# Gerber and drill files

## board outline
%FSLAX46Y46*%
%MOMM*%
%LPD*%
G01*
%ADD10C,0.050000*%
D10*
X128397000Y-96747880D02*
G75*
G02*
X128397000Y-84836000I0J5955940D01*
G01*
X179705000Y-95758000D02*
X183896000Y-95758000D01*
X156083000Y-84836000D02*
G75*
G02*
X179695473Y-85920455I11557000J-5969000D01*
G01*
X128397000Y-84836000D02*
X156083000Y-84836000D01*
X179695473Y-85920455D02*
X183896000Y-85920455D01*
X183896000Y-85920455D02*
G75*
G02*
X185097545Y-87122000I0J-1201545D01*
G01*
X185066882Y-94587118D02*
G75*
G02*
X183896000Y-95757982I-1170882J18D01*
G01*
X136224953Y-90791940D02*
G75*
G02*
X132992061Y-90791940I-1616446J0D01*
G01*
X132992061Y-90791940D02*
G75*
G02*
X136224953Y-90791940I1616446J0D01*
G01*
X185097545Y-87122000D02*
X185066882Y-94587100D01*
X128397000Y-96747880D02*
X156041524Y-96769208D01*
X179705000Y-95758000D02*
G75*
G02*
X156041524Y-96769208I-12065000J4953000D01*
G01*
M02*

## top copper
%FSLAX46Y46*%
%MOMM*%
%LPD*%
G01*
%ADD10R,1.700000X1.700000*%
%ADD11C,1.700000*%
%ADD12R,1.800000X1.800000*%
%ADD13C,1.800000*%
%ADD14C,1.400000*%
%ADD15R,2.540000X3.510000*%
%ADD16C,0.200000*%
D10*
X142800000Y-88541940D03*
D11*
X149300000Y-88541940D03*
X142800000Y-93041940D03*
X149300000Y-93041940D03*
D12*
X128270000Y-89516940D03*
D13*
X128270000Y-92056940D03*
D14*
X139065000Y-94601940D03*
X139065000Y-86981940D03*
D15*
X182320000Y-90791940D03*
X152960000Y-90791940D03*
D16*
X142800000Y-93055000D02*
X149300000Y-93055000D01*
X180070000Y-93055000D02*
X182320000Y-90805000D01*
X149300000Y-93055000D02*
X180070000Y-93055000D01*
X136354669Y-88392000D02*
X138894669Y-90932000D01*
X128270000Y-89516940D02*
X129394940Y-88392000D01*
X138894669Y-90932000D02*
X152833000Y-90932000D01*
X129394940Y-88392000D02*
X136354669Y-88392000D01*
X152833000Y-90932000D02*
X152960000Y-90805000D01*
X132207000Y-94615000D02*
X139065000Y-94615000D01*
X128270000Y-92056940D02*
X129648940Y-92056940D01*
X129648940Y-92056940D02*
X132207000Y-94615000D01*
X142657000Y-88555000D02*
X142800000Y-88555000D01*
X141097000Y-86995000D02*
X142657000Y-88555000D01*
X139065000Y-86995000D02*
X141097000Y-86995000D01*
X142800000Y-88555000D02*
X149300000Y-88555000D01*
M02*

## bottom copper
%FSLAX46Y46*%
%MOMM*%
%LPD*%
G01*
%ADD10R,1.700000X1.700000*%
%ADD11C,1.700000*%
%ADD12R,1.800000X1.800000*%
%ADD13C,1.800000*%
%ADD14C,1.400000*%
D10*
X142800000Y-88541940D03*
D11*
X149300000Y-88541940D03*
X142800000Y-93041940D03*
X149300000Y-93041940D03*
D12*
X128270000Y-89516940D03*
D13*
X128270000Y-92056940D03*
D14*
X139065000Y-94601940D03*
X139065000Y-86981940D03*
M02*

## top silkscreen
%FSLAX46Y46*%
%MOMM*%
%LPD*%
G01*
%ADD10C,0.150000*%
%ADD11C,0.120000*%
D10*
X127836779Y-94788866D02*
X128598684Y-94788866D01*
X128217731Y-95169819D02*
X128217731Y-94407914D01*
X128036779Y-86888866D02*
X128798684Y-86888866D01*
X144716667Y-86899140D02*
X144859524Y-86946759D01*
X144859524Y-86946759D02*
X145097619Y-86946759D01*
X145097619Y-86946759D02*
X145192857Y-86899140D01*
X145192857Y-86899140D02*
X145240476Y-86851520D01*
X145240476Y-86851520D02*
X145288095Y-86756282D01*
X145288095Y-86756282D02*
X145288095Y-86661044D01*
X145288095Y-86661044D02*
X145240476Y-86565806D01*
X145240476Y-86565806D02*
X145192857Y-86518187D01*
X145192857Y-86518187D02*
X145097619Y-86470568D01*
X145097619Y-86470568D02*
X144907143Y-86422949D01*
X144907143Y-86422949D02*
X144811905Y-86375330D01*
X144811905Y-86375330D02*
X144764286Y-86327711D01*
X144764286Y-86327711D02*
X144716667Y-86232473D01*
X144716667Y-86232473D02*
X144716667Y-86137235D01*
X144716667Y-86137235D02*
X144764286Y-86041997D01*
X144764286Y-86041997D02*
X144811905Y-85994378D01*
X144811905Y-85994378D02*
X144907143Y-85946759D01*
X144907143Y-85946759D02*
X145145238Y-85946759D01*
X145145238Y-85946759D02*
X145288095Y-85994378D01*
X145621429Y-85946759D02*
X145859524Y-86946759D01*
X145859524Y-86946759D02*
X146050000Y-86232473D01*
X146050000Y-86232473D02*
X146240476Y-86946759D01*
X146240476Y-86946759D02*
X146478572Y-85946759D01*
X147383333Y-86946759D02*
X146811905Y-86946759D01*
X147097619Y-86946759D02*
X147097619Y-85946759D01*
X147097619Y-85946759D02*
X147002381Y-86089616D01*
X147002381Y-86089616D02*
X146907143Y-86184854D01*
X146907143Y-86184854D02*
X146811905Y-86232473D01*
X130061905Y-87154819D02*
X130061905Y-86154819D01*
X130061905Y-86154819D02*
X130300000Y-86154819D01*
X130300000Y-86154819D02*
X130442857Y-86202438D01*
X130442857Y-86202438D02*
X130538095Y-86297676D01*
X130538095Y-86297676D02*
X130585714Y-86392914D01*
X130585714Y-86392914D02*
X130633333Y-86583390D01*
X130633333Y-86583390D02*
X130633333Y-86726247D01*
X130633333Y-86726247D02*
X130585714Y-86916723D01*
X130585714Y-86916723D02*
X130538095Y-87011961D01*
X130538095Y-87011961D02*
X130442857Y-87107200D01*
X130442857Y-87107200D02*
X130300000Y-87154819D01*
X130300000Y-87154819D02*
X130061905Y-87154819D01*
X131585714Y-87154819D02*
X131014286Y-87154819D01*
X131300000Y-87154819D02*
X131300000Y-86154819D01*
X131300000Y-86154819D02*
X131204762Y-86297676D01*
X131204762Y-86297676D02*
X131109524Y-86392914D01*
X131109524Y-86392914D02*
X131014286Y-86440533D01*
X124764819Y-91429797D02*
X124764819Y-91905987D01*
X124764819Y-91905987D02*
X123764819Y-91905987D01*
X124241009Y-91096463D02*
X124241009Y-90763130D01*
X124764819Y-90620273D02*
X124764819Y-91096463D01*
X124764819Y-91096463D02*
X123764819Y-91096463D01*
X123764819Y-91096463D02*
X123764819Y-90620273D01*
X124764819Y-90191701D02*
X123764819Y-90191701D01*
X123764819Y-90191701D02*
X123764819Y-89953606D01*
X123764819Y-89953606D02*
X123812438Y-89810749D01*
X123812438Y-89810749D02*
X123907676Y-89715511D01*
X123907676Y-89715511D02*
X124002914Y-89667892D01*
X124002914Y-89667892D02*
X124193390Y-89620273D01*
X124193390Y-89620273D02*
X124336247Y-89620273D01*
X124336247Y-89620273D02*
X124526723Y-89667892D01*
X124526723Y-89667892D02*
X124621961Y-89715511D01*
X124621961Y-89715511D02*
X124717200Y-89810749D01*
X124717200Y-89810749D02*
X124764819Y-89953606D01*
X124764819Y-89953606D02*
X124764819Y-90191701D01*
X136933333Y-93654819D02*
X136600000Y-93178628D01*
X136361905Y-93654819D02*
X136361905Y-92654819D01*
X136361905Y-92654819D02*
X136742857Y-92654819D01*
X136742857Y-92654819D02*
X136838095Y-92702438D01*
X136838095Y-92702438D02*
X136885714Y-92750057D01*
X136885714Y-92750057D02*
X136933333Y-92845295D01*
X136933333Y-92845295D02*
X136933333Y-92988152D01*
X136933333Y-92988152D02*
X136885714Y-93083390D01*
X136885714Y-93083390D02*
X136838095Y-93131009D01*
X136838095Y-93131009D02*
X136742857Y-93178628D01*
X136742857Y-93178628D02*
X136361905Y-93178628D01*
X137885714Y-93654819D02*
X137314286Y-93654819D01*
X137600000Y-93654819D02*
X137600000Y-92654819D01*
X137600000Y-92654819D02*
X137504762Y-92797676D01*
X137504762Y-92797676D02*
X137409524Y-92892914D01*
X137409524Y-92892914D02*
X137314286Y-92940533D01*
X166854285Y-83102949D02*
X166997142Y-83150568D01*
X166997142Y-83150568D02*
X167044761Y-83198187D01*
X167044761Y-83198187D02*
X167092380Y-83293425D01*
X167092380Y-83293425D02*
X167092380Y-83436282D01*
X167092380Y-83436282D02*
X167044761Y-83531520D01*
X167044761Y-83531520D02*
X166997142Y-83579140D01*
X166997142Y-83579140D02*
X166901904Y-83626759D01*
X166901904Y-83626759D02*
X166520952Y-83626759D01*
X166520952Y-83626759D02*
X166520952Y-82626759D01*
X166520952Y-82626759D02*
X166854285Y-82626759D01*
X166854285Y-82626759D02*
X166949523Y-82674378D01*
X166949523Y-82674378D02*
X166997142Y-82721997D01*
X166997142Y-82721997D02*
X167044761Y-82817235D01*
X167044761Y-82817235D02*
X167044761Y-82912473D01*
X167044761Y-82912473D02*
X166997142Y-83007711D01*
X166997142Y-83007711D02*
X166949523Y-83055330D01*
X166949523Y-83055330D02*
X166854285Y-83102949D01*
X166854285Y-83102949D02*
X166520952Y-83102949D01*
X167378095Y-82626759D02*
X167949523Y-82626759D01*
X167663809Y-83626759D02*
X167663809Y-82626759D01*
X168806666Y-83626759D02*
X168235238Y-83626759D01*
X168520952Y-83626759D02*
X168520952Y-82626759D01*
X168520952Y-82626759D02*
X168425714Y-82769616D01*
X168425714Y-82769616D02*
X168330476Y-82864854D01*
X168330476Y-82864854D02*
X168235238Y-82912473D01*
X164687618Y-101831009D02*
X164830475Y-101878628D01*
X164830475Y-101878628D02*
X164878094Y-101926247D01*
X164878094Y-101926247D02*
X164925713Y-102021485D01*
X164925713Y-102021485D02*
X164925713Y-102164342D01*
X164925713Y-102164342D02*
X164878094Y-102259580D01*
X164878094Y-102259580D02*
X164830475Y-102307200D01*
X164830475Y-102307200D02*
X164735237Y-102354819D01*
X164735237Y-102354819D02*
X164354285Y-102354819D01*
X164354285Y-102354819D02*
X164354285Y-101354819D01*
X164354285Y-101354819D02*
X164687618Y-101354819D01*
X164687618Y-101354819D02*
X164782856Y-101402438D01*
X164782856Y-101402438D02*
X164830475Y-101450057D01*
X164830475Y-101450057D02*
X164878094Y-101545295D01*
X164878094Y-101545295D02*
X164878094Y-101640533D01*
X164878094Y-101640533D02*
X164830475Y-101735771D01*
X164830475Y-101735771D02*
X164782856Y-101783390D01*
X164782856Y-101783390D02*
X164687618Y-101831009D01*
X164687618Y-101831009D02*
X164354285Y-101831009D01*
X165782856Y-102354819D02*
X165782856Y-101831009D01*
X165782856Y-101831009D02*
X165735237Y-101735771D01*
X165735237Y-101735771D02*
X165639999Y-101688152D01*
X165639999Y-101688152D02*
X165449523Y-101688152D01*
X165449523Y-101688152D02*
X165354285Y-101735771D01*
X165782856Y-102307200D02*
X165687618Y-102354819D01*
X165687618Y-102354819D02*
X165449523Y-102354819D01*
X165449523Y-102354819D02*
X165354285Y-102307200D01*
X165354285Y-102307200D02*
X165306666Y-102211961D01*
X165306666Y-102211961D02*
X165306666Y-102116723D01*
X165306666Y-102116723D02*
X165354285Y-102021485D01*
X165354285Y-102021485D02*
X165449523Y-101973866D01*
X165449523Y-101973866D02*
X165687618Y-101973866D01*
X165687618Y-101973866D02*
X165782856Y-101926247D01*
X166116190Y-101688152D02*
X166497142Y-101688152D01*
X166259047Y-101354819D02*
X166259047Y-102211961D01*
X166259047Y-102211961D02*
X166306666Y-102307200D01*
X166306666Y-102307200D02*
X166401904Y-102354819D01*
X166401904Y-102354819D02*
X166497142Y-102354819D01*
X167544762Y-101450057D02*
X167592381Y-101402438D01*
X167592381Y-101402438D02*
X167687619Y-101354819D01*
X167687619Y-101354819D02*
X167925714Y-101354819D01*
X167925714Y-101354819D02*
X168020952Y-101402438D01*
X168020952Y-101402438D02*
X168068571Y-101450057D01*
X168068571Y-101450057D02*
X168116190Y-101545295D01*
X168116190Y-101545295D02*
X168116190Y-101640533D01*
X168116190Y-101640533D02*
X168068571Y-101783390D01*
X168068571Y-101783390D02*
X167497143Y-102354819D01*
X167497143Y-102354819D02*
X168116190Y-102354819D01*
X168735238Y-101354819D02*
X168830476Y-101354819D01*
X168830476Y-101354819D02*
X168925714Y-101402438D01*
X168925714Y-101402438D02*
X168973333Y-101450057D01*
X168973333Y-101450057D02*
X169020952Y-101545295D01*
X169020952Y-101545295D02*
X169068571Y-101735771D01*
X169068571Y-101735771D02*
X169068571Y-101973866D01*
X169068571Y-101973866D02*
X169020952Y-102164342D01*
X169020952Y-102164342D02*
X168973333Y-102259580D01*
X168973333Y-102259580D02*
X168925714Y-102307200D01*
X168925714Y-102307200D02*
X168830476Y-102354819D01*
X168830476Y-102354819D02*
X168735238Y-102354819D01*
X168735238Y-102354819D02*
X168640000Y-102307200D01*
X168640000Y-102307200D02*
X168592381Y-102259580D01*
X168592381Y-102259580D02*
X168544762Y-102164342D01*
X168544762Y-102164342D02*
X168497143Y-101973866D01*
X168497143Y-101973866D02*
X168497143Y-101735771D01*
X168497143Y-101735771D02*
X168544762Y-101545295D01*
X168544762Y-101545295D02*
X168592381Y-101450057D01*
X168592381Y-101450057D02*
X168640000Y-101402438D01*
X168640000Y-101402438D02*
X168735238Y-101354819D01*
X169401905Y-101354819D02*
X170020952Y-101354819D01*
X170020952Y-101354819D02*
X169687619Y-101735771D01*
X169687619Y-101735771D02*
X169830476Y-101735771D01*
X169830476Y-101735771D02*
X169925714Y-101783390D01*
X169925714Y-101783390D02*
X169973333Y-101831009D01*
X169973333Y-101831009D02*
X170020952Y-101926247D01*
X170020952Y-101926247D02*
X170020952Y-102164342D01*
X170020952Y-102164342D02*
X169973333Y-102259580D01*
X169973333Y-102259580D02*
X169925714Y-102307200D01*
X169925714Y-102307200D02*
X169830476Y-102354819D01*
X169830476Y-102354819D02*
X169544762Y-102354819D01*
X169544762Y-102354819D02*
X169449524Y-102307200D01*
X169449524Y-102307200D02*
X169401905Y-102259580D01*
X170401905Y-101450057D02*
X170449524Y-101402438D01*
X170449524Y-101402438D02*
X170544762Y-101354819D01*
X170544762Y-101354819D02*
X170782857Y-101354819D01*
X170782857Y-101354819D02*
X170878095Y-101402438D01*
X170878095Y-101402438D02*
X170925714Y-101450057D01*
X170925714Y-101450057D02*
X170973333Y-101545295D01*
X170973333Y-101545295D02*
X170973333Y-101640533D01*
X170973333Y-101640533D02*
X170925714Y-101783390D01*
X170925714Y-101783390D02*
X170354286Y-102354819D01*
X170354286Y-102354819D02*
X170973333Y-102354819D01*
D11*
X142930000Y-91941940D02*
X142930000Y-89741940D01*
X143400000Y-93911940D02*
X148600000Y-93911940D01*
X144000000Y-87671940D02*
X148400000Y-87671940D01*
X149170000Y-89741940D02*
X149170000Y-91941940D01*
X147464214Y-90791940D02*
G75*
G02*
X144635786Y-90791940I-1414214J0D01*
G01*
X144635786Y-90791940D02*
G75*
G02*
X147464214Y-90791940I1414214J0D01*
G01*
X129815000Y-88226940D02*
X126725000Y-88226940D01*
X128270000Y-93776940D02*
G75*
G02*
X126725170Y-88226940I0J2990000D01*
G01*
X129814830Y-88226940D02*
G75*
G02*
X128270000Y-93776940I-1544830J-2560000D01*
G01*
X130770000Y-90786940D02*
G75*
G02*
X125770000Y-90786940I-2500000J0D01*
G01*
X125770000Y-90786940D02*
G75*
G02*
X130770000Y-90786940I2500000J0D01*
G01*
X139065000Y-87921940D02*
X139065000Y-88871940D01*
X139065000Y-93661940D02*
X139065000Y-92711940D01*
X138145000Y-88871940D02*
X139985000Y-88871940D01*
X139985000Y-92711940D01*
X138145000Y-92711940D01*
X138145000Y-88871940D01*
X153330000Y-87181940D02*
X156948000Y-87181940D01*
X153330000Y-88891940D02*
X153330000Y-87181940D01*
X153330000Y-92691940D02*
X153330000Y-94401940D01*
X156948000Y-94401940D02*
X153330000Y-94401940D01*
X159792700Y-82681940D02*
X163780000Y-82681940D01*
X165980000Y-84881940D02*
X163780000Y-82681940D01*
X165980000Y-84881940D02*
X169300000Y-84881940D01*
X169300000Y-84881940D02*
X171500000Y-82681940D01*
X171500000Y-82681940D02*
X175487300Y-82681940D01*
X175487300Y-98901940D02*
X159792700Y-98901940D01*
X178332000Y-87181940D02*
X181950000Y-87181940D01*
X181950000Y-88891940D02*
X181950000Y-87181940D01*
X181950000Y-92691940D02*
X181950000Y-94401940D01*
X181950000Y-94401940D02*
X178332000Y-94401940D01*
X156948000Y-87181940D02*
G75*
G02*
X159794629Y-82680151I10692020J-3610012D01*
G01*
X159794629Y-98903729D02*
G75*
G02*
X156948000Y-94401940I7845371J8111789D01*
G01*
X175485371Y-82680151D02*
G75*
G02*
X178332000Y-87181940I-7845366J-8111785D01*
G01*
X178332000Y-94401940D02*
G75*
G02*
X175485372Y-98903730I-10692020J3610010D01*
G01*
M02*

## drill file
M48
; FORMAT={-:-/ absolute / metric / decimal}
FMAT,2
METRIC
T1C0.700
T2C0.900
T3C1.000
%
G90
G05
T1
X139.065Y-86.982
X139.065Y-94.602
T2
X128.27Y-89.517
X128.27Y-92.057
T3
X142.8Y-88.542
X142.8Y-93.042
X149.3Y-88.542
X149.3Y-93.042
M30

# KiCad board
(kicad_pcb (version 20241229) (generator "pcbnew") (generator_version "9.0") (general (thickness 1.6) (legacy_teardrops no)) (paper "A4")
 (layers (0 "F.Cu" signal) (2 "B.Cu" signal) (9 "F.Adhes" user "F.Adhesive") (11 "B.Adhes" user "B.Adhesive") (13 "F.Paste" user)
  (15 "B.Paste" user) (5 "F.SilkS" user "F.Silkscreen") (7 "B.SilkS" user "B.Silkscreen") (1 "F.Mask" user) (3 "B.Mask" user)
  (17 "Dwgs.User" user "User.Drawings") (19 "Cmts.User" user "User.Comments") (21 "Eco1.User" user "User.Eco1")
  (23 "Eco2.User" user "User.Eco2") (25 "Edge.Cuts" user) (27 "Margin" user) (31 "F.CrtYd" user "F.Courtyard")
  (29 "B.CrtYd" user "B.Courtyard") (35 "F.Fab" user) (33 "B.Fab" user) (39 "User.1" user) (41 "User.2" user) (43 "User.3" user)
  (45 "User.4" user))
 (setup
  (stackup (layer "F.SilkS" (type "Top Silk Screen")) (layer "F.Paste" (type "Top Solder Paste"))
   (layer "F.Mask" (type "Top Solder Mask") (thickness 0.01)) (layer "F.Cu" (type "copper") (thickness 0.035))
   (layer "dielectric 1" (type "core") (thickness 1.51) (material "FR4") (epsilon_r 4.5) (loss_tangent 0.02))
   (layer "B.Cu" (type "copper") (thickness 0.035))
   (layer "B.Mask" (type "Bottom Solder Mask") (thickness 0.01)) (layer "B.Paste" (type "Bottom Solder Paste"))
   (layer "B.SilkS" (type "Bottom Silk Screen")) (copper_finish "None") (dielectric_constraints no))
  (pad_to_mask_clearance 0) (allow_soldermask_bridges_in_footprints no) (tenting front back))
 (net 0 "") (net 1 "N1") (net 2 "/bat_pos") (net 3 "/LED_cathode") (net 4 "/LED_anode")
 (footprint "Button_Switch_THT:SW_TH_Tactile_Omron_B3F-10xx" (layer "F.Cu") (at 142.8 88.54194)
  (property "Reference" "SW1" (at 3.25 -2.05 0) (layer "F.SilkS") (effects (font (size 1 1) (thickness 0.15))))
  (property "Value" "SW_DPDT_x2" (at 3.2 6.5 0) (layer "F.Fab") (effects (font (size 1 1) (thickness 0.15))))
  (fp_line (start 0.13 3.4) (end 0.13 1.2) (stroke (width 0.12) (type solid)) (layer "F.SilkS"))
  (fp_line (start 0.6 5.37) (end 5.8 5.37) (stroke (width 0.12) (type solid)) (layer "F.SilkS"))
  (fp_line (start 1.2 -0.87) (end 5.6 -0.87) (stroke (width 0.12) (type solid)) (layer "F.SilkS"))
  (fp_line (start 6.37 1.2) (end 6.37 3.4) (stroke (width 0.12) (type solid)) (layer "F.SilkS"))
  (fp_circle (center 3.25 2.25) (end 4.25 3.25) (stroke (width 0.12) (type solid)) (fill no) (layer "F.SilkS"))
  (pad "1" thru_hole rect (at 0 0) (size 1.7 1.7) (drill 1) (layers "*.Cu" "*.Mask") (remove_unused_layers no) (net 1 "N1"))
  (pad "1" thru_hole circle (at 6.5 0) (size 1.7 1.7) (drill 1) (layers "*.Cu" "*.Mask") (remove_unused_layers no) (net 1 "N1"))
  (pad "2" thru_hole circle (at 0 4.5) (size 1.7 1.7) (drill 1) (layers "*.Cu" "*.Mask") (remove_unused_layers no) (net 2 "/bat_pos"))
  (pad "2" thru_hole circle (at 6.5 4.5) (size 1.7 1.7) (drill 1) (layers "*.Cu" "*.Mask") (remove_unused_layers no) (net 2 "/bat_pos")))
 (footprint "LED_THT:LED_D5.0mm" (layer "F.Cu") (at 128.27 89.51694 -90)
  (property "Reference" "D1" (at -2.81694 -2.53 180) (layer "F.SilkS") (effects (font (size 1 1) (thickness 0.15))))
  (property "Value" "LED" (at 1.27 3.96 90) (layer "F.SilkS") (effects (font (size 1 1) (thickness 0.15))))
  (fp_line (start -1.29 -1.545) (end -1.29 1.545) (stroke (width 0.12) (type solid)) (layer "F.SilkS"))
  (fp_arc (start 4.26 0) (mid 2.071779 2.880495) (end -1.29 1.54483) (stroke (width 0.12) (type solid)) (layer "F.SilkS"))
  (fp_arc (start -1.29 -1.54483) (mid 2.071779 -2.880495) (end 4.26 0) (stroke (width 0.12) (type solid)) (layer "F.SilkS"))
  (fp_circle (center 1.27 0) (end 3.77 0) (stroke (width 0.12) (type solid)) (fill no) (layer "F.SilkS"))
  (pad "1" thru_hole rect (at 0 0 270) (size 1.8 1.8) (drill 0.9) (layers "*.Cu" "*.Mask") (remove_unused_layers no) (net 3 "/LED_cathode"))
  (pad "2" thru_hole circle (at 2.54 0 270) (size 1.8 1.8) (drill 0.9) (layers "*.Cu" "*.Mask") (remove_unused_layers no)
   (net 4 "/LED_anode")))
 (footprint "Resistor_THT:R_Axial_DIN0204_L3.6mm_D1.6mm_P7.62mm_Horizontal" (layer "F.Cu") (at 139.065 94.60194 90)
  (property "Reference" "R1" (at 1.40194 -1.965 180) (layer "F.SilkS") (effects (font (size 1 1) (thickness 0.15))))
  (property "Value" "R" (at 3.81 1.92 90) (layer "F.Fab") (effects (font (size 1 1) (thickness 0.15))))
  (fp_line (start 6.68 0) (end 5.73 0) (stroke (width 0.12) (type solid)) (layer "F.SilkS"))
  (fp_line (start 0.94 0) (end 1.89 0) (stroke (width 0.12) (type solid)) (layer "F.SilkS"))
  (fp_rect (start 1.89 -0.92) (end 5.73 0.92) (stroke (width 0.12) (type solid)) (fill no) (layer "F.SilkS"))
  (pad "1" thru_hole circle (at 0 0 90) (size 1.4 1.4) (drill 0.7) (layers "*.Cu" "*.Mask") (remove_unused_layers no) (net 4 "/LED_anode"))
  (pad "2" thru_hole circle (at 7.62 0 90) (size 1.4 1.4) (drill 0.7) (layers "*.Cu" "*.Mask") (remove_unused_layers no) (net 1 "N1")))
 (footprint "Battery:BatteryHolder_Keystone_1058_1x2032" (layer "F.Cu") (at 167.64 90.79194 180)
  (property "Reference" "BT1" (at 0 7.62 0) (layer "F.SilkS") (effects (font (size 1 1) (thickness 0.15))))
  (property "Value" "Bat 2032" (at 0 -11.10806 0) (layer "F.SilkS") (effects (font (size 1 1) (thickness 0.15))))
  (fp_line (start 14.31 3.61) (end 10.692 3.61) (stroke (width 0.12) (type solid)) (layer "F.SilkS"))
  (fp_line (start 14.31 1.9) (end 14.31 3.61) (stroke (width 0.12) (type solid)) (layer "F.SilkS"))
  (fp_line (start 14.31 -1.9) (end 14.31 -3.61) (stroke (width 0.12) (type solid)) (layer "F.SilkS"))
  (fp_line (start 10.692 -3.61) (end 14.31 -3.61) (stroke (width 0.12) (type solid)) (layer "F.SilkS"))
  (fp_line (start 7.8473 8.11) (end 3.86 8.11) (stroke (width 0.12) (type solid)) (layer "F.SilkS"))
  (fp_line (start 1.66 5.91) (end 3.86 8.11) (stroke (width 0.12) (type solid)) (layer "F.SilkS"))
  (fp_line (start 1.66 5.91) (end -1.66 5.91) (stroke (width 0.12) (type solid)) (layer "F.SilkS"))
  (fp_line (start -1.66 5.91) (end -3.86 8.11) (stroke (width 0.12) (type solid)) (layer "F.SilkS"))
  (fp_line (start -3.86 8.11) (end -7.8473 8.11) (stroke (width 0.12) (type solid)) (layer "F.SilkS"))
  (fp_line (start -7.8473 -8.11) (end 7.8473 -8.11) (stroke (width 0.12) (type solid)) (layer "F.SilkS"))
  (fp_line (start -10.692 3.61) (end -14.31 3.61) (stroke (width 0.12) (type solid)) (layer "F.SilkS"))
  (fp_line (start -14.31 1.9) (end -14.31 3.61) (stroke (width 0.12) (type solid)) (layer "F.SilkS"))
  (fp_line (start -14.31 -1.9) (end -14.31 -3.61) (stroke (width 0.12) (type solid)) (layer "F.SilkS"))
  (fp_line (start -14.31 -3.61) (end -10.692 -3.61) (stroke (width 0.12) (type solid)) (layer "F.SilkS"))
  (fp_arc (start 10.692 3.61) (mid 9.538084 6.031244) (end 7.845371 8.111789) (stroke (width 0.12) (type solid)) (layer "F.SilkS"))
  (fp_arc (start 7.845371 -8.111789) (mid 9.538085 -6.031244) (end 10.692 -3.61) (stroke (width 0.12) (type solid)) (layer "F.SilkS"))
  (fp_arc (start -7.845371 8.111789) (mid -9.538085 6.031244) (end -10.692 3.61) (stroke (width 0.12) (type solid)) (layer "F.SilkS"))
  (fp_arc (start -10.692 -3.61) (mid -9.538084 -6.031244) (end -7.845371 -8.111789) (stroke (width 0.12) (type solid)) (layer "F.SilkS"))
  (pad "1" smd rect (at -14.68 0 180) (size 2.54 3.51) (layers "F.Cu" "F.Mask" "F.Paste") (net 2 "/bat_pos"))
  (pad "2" smd rect (at 14.68 0 180) (size 2.54 3.51) (layers "F.Cu" "F.Mask" "F.Paste") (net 3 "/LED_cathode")))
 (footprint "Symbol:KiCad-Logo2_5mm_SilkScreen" (layer "B.Cu") (at 167.767 87.63 180)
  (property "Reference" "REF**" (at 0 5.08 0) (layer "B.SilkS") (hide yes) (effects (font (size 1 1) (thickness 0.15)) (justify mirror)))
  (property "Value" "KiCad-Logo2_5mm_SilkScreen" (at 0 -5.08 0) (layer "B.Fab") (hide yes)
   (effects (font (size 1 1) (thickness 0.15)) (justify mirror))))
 (gr_arc (start 128.397 96.74788) (mid 122.44106 90.79194) (end 128.397 84.836) (stroke (width 0.05) (type default)) (locked yes)
  (layer "Edge.Cuts"))
 (gr_line (start 179.705 95.758) (end 183.896 95.758) (stroke (width 0.05) (type default)) (locked yes) (layer "Edge.Cuts"))
 (gr_arc (start 156.083 84.836) (mid 168.236766 77.811268) (end 179.695473 85.920455) (stroke (width 0.05) (type default)) (locked yes)
  (layer "Edge.Cuts"))
 (gr_line (start 128.397 84.836) (end 156.083 84.836) (stroke (width 0.05) (type default)) (locked yes) (layer "Edge.Cuts"))
 (gr_line (start 179.695473 85.920455) (end 183.896 85.920455) (stroke (width 0.05) (type default)) (locked yes) (layer "Edge.Cuts"))
 (gr_arc (start 183.896 85.920455) (mid 184.745621 86.272379) (end 185.097545 87.122) (stroke (width 0.05) (type default)) (locked yes)
  (layer "Edge.Cuts"))
 (gr_arc (start 185.066882 94.587118) (mid 184.723939 95.415057) (end 183.896 95.758) (stroke (width 0.05) (type default)) (locked yes)
  (layer "Edge.Cuts"))
 (gr_circle (center 134.608507 90.79194) (end 135.751507 91.93494) (stroke (width 0.05) (type default)) (fill no) (layer "Edge.Cuts"))
 (gr_line (start 185.097545 87.122) (end 185.066882 94.5871) (stroke (width 0.05) (type default)) (locked yes) (layer "Edge.Cuts"))
 (gr_line (start 128.397 96.74788) (end 156.041524 96.769208) (stroke (width 0.05) (type default)) (locked yes) (layer "Edge.Cuts"))
 (gr_arc (start 179.705 95.758) (mid 168.196818 103.835211) (end 156.041524 96.769208) (stroke (width 0.05) (type default)) (locked yes)
  (layer "Edge.Cuts"))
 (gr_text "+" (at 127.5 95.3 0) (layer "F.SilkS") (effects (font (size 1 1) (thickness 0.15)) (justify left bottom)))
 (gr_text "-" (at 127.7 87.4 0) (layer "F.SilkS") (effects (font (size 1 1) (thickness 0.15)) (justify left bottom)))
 (segment (start 142.8 93.055) (end 149.3 93.055) (width 0.2) (layer "F.Cu") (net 2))
 (segment (start 180.07 93.055) (end 182.32 90.805) (width 0.2) (layer "F.Cu") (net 2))
 (segment (start 149.3 93.055) (end 180.07 93.055) (width 0.2) (layer "F.Cu") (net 2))
 (segment (start 136.354669 88.392) (end 138.894669 90.932) (width 0.2) (layer "F.Cu") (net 3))
 (segment (start 128.27 89.51694) (end 129.39494 88.392) (width 0.2) (layer "F.Cu") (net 3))
 (segment (start 138.894669 90.932) (end 152.833 90.932) (width 0.2) (layer "F.Cu") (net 3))
 (segment (start 129.39494 88.392) (end 136.354669 88.392) (width 0.2) (layer "F.Cu") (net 3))
 (segment (start 152.833 90.932) (end 152.96 90.805) (width 0.2) (layer "F.Cu") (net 3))
 (segment (start 132.207 94.615) (end 139.065 94.615) (width 0.2) (layer "F.Cu") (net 4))
 (segment (start 128.27 92.05694) (end 129.64894 92.05694) (width 0.2) (layer "F.Cu") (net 4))
 (segment (start 129.64894 92.05694) (end 132.207 94.615) (width 0.2) (layer "F.Cu") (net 4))
 (segment (start 142.657 88.555) (end 142.8 88.555) (width 0.2) (layer "F.Cu") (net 1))
 (segment (start 141.097 86.995) (end 142.657 88.555) (width 0.2) (layer "F.Cu") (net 1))
 (segment (start 139.065 86.995) (end 141.097 86.995) (width 0.2) (layer "F.Cu") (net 1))
 (segment (start 142.8 88.555) (end 149.3 88.555) (width 0.2) (layer "F.Cu") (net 1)))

